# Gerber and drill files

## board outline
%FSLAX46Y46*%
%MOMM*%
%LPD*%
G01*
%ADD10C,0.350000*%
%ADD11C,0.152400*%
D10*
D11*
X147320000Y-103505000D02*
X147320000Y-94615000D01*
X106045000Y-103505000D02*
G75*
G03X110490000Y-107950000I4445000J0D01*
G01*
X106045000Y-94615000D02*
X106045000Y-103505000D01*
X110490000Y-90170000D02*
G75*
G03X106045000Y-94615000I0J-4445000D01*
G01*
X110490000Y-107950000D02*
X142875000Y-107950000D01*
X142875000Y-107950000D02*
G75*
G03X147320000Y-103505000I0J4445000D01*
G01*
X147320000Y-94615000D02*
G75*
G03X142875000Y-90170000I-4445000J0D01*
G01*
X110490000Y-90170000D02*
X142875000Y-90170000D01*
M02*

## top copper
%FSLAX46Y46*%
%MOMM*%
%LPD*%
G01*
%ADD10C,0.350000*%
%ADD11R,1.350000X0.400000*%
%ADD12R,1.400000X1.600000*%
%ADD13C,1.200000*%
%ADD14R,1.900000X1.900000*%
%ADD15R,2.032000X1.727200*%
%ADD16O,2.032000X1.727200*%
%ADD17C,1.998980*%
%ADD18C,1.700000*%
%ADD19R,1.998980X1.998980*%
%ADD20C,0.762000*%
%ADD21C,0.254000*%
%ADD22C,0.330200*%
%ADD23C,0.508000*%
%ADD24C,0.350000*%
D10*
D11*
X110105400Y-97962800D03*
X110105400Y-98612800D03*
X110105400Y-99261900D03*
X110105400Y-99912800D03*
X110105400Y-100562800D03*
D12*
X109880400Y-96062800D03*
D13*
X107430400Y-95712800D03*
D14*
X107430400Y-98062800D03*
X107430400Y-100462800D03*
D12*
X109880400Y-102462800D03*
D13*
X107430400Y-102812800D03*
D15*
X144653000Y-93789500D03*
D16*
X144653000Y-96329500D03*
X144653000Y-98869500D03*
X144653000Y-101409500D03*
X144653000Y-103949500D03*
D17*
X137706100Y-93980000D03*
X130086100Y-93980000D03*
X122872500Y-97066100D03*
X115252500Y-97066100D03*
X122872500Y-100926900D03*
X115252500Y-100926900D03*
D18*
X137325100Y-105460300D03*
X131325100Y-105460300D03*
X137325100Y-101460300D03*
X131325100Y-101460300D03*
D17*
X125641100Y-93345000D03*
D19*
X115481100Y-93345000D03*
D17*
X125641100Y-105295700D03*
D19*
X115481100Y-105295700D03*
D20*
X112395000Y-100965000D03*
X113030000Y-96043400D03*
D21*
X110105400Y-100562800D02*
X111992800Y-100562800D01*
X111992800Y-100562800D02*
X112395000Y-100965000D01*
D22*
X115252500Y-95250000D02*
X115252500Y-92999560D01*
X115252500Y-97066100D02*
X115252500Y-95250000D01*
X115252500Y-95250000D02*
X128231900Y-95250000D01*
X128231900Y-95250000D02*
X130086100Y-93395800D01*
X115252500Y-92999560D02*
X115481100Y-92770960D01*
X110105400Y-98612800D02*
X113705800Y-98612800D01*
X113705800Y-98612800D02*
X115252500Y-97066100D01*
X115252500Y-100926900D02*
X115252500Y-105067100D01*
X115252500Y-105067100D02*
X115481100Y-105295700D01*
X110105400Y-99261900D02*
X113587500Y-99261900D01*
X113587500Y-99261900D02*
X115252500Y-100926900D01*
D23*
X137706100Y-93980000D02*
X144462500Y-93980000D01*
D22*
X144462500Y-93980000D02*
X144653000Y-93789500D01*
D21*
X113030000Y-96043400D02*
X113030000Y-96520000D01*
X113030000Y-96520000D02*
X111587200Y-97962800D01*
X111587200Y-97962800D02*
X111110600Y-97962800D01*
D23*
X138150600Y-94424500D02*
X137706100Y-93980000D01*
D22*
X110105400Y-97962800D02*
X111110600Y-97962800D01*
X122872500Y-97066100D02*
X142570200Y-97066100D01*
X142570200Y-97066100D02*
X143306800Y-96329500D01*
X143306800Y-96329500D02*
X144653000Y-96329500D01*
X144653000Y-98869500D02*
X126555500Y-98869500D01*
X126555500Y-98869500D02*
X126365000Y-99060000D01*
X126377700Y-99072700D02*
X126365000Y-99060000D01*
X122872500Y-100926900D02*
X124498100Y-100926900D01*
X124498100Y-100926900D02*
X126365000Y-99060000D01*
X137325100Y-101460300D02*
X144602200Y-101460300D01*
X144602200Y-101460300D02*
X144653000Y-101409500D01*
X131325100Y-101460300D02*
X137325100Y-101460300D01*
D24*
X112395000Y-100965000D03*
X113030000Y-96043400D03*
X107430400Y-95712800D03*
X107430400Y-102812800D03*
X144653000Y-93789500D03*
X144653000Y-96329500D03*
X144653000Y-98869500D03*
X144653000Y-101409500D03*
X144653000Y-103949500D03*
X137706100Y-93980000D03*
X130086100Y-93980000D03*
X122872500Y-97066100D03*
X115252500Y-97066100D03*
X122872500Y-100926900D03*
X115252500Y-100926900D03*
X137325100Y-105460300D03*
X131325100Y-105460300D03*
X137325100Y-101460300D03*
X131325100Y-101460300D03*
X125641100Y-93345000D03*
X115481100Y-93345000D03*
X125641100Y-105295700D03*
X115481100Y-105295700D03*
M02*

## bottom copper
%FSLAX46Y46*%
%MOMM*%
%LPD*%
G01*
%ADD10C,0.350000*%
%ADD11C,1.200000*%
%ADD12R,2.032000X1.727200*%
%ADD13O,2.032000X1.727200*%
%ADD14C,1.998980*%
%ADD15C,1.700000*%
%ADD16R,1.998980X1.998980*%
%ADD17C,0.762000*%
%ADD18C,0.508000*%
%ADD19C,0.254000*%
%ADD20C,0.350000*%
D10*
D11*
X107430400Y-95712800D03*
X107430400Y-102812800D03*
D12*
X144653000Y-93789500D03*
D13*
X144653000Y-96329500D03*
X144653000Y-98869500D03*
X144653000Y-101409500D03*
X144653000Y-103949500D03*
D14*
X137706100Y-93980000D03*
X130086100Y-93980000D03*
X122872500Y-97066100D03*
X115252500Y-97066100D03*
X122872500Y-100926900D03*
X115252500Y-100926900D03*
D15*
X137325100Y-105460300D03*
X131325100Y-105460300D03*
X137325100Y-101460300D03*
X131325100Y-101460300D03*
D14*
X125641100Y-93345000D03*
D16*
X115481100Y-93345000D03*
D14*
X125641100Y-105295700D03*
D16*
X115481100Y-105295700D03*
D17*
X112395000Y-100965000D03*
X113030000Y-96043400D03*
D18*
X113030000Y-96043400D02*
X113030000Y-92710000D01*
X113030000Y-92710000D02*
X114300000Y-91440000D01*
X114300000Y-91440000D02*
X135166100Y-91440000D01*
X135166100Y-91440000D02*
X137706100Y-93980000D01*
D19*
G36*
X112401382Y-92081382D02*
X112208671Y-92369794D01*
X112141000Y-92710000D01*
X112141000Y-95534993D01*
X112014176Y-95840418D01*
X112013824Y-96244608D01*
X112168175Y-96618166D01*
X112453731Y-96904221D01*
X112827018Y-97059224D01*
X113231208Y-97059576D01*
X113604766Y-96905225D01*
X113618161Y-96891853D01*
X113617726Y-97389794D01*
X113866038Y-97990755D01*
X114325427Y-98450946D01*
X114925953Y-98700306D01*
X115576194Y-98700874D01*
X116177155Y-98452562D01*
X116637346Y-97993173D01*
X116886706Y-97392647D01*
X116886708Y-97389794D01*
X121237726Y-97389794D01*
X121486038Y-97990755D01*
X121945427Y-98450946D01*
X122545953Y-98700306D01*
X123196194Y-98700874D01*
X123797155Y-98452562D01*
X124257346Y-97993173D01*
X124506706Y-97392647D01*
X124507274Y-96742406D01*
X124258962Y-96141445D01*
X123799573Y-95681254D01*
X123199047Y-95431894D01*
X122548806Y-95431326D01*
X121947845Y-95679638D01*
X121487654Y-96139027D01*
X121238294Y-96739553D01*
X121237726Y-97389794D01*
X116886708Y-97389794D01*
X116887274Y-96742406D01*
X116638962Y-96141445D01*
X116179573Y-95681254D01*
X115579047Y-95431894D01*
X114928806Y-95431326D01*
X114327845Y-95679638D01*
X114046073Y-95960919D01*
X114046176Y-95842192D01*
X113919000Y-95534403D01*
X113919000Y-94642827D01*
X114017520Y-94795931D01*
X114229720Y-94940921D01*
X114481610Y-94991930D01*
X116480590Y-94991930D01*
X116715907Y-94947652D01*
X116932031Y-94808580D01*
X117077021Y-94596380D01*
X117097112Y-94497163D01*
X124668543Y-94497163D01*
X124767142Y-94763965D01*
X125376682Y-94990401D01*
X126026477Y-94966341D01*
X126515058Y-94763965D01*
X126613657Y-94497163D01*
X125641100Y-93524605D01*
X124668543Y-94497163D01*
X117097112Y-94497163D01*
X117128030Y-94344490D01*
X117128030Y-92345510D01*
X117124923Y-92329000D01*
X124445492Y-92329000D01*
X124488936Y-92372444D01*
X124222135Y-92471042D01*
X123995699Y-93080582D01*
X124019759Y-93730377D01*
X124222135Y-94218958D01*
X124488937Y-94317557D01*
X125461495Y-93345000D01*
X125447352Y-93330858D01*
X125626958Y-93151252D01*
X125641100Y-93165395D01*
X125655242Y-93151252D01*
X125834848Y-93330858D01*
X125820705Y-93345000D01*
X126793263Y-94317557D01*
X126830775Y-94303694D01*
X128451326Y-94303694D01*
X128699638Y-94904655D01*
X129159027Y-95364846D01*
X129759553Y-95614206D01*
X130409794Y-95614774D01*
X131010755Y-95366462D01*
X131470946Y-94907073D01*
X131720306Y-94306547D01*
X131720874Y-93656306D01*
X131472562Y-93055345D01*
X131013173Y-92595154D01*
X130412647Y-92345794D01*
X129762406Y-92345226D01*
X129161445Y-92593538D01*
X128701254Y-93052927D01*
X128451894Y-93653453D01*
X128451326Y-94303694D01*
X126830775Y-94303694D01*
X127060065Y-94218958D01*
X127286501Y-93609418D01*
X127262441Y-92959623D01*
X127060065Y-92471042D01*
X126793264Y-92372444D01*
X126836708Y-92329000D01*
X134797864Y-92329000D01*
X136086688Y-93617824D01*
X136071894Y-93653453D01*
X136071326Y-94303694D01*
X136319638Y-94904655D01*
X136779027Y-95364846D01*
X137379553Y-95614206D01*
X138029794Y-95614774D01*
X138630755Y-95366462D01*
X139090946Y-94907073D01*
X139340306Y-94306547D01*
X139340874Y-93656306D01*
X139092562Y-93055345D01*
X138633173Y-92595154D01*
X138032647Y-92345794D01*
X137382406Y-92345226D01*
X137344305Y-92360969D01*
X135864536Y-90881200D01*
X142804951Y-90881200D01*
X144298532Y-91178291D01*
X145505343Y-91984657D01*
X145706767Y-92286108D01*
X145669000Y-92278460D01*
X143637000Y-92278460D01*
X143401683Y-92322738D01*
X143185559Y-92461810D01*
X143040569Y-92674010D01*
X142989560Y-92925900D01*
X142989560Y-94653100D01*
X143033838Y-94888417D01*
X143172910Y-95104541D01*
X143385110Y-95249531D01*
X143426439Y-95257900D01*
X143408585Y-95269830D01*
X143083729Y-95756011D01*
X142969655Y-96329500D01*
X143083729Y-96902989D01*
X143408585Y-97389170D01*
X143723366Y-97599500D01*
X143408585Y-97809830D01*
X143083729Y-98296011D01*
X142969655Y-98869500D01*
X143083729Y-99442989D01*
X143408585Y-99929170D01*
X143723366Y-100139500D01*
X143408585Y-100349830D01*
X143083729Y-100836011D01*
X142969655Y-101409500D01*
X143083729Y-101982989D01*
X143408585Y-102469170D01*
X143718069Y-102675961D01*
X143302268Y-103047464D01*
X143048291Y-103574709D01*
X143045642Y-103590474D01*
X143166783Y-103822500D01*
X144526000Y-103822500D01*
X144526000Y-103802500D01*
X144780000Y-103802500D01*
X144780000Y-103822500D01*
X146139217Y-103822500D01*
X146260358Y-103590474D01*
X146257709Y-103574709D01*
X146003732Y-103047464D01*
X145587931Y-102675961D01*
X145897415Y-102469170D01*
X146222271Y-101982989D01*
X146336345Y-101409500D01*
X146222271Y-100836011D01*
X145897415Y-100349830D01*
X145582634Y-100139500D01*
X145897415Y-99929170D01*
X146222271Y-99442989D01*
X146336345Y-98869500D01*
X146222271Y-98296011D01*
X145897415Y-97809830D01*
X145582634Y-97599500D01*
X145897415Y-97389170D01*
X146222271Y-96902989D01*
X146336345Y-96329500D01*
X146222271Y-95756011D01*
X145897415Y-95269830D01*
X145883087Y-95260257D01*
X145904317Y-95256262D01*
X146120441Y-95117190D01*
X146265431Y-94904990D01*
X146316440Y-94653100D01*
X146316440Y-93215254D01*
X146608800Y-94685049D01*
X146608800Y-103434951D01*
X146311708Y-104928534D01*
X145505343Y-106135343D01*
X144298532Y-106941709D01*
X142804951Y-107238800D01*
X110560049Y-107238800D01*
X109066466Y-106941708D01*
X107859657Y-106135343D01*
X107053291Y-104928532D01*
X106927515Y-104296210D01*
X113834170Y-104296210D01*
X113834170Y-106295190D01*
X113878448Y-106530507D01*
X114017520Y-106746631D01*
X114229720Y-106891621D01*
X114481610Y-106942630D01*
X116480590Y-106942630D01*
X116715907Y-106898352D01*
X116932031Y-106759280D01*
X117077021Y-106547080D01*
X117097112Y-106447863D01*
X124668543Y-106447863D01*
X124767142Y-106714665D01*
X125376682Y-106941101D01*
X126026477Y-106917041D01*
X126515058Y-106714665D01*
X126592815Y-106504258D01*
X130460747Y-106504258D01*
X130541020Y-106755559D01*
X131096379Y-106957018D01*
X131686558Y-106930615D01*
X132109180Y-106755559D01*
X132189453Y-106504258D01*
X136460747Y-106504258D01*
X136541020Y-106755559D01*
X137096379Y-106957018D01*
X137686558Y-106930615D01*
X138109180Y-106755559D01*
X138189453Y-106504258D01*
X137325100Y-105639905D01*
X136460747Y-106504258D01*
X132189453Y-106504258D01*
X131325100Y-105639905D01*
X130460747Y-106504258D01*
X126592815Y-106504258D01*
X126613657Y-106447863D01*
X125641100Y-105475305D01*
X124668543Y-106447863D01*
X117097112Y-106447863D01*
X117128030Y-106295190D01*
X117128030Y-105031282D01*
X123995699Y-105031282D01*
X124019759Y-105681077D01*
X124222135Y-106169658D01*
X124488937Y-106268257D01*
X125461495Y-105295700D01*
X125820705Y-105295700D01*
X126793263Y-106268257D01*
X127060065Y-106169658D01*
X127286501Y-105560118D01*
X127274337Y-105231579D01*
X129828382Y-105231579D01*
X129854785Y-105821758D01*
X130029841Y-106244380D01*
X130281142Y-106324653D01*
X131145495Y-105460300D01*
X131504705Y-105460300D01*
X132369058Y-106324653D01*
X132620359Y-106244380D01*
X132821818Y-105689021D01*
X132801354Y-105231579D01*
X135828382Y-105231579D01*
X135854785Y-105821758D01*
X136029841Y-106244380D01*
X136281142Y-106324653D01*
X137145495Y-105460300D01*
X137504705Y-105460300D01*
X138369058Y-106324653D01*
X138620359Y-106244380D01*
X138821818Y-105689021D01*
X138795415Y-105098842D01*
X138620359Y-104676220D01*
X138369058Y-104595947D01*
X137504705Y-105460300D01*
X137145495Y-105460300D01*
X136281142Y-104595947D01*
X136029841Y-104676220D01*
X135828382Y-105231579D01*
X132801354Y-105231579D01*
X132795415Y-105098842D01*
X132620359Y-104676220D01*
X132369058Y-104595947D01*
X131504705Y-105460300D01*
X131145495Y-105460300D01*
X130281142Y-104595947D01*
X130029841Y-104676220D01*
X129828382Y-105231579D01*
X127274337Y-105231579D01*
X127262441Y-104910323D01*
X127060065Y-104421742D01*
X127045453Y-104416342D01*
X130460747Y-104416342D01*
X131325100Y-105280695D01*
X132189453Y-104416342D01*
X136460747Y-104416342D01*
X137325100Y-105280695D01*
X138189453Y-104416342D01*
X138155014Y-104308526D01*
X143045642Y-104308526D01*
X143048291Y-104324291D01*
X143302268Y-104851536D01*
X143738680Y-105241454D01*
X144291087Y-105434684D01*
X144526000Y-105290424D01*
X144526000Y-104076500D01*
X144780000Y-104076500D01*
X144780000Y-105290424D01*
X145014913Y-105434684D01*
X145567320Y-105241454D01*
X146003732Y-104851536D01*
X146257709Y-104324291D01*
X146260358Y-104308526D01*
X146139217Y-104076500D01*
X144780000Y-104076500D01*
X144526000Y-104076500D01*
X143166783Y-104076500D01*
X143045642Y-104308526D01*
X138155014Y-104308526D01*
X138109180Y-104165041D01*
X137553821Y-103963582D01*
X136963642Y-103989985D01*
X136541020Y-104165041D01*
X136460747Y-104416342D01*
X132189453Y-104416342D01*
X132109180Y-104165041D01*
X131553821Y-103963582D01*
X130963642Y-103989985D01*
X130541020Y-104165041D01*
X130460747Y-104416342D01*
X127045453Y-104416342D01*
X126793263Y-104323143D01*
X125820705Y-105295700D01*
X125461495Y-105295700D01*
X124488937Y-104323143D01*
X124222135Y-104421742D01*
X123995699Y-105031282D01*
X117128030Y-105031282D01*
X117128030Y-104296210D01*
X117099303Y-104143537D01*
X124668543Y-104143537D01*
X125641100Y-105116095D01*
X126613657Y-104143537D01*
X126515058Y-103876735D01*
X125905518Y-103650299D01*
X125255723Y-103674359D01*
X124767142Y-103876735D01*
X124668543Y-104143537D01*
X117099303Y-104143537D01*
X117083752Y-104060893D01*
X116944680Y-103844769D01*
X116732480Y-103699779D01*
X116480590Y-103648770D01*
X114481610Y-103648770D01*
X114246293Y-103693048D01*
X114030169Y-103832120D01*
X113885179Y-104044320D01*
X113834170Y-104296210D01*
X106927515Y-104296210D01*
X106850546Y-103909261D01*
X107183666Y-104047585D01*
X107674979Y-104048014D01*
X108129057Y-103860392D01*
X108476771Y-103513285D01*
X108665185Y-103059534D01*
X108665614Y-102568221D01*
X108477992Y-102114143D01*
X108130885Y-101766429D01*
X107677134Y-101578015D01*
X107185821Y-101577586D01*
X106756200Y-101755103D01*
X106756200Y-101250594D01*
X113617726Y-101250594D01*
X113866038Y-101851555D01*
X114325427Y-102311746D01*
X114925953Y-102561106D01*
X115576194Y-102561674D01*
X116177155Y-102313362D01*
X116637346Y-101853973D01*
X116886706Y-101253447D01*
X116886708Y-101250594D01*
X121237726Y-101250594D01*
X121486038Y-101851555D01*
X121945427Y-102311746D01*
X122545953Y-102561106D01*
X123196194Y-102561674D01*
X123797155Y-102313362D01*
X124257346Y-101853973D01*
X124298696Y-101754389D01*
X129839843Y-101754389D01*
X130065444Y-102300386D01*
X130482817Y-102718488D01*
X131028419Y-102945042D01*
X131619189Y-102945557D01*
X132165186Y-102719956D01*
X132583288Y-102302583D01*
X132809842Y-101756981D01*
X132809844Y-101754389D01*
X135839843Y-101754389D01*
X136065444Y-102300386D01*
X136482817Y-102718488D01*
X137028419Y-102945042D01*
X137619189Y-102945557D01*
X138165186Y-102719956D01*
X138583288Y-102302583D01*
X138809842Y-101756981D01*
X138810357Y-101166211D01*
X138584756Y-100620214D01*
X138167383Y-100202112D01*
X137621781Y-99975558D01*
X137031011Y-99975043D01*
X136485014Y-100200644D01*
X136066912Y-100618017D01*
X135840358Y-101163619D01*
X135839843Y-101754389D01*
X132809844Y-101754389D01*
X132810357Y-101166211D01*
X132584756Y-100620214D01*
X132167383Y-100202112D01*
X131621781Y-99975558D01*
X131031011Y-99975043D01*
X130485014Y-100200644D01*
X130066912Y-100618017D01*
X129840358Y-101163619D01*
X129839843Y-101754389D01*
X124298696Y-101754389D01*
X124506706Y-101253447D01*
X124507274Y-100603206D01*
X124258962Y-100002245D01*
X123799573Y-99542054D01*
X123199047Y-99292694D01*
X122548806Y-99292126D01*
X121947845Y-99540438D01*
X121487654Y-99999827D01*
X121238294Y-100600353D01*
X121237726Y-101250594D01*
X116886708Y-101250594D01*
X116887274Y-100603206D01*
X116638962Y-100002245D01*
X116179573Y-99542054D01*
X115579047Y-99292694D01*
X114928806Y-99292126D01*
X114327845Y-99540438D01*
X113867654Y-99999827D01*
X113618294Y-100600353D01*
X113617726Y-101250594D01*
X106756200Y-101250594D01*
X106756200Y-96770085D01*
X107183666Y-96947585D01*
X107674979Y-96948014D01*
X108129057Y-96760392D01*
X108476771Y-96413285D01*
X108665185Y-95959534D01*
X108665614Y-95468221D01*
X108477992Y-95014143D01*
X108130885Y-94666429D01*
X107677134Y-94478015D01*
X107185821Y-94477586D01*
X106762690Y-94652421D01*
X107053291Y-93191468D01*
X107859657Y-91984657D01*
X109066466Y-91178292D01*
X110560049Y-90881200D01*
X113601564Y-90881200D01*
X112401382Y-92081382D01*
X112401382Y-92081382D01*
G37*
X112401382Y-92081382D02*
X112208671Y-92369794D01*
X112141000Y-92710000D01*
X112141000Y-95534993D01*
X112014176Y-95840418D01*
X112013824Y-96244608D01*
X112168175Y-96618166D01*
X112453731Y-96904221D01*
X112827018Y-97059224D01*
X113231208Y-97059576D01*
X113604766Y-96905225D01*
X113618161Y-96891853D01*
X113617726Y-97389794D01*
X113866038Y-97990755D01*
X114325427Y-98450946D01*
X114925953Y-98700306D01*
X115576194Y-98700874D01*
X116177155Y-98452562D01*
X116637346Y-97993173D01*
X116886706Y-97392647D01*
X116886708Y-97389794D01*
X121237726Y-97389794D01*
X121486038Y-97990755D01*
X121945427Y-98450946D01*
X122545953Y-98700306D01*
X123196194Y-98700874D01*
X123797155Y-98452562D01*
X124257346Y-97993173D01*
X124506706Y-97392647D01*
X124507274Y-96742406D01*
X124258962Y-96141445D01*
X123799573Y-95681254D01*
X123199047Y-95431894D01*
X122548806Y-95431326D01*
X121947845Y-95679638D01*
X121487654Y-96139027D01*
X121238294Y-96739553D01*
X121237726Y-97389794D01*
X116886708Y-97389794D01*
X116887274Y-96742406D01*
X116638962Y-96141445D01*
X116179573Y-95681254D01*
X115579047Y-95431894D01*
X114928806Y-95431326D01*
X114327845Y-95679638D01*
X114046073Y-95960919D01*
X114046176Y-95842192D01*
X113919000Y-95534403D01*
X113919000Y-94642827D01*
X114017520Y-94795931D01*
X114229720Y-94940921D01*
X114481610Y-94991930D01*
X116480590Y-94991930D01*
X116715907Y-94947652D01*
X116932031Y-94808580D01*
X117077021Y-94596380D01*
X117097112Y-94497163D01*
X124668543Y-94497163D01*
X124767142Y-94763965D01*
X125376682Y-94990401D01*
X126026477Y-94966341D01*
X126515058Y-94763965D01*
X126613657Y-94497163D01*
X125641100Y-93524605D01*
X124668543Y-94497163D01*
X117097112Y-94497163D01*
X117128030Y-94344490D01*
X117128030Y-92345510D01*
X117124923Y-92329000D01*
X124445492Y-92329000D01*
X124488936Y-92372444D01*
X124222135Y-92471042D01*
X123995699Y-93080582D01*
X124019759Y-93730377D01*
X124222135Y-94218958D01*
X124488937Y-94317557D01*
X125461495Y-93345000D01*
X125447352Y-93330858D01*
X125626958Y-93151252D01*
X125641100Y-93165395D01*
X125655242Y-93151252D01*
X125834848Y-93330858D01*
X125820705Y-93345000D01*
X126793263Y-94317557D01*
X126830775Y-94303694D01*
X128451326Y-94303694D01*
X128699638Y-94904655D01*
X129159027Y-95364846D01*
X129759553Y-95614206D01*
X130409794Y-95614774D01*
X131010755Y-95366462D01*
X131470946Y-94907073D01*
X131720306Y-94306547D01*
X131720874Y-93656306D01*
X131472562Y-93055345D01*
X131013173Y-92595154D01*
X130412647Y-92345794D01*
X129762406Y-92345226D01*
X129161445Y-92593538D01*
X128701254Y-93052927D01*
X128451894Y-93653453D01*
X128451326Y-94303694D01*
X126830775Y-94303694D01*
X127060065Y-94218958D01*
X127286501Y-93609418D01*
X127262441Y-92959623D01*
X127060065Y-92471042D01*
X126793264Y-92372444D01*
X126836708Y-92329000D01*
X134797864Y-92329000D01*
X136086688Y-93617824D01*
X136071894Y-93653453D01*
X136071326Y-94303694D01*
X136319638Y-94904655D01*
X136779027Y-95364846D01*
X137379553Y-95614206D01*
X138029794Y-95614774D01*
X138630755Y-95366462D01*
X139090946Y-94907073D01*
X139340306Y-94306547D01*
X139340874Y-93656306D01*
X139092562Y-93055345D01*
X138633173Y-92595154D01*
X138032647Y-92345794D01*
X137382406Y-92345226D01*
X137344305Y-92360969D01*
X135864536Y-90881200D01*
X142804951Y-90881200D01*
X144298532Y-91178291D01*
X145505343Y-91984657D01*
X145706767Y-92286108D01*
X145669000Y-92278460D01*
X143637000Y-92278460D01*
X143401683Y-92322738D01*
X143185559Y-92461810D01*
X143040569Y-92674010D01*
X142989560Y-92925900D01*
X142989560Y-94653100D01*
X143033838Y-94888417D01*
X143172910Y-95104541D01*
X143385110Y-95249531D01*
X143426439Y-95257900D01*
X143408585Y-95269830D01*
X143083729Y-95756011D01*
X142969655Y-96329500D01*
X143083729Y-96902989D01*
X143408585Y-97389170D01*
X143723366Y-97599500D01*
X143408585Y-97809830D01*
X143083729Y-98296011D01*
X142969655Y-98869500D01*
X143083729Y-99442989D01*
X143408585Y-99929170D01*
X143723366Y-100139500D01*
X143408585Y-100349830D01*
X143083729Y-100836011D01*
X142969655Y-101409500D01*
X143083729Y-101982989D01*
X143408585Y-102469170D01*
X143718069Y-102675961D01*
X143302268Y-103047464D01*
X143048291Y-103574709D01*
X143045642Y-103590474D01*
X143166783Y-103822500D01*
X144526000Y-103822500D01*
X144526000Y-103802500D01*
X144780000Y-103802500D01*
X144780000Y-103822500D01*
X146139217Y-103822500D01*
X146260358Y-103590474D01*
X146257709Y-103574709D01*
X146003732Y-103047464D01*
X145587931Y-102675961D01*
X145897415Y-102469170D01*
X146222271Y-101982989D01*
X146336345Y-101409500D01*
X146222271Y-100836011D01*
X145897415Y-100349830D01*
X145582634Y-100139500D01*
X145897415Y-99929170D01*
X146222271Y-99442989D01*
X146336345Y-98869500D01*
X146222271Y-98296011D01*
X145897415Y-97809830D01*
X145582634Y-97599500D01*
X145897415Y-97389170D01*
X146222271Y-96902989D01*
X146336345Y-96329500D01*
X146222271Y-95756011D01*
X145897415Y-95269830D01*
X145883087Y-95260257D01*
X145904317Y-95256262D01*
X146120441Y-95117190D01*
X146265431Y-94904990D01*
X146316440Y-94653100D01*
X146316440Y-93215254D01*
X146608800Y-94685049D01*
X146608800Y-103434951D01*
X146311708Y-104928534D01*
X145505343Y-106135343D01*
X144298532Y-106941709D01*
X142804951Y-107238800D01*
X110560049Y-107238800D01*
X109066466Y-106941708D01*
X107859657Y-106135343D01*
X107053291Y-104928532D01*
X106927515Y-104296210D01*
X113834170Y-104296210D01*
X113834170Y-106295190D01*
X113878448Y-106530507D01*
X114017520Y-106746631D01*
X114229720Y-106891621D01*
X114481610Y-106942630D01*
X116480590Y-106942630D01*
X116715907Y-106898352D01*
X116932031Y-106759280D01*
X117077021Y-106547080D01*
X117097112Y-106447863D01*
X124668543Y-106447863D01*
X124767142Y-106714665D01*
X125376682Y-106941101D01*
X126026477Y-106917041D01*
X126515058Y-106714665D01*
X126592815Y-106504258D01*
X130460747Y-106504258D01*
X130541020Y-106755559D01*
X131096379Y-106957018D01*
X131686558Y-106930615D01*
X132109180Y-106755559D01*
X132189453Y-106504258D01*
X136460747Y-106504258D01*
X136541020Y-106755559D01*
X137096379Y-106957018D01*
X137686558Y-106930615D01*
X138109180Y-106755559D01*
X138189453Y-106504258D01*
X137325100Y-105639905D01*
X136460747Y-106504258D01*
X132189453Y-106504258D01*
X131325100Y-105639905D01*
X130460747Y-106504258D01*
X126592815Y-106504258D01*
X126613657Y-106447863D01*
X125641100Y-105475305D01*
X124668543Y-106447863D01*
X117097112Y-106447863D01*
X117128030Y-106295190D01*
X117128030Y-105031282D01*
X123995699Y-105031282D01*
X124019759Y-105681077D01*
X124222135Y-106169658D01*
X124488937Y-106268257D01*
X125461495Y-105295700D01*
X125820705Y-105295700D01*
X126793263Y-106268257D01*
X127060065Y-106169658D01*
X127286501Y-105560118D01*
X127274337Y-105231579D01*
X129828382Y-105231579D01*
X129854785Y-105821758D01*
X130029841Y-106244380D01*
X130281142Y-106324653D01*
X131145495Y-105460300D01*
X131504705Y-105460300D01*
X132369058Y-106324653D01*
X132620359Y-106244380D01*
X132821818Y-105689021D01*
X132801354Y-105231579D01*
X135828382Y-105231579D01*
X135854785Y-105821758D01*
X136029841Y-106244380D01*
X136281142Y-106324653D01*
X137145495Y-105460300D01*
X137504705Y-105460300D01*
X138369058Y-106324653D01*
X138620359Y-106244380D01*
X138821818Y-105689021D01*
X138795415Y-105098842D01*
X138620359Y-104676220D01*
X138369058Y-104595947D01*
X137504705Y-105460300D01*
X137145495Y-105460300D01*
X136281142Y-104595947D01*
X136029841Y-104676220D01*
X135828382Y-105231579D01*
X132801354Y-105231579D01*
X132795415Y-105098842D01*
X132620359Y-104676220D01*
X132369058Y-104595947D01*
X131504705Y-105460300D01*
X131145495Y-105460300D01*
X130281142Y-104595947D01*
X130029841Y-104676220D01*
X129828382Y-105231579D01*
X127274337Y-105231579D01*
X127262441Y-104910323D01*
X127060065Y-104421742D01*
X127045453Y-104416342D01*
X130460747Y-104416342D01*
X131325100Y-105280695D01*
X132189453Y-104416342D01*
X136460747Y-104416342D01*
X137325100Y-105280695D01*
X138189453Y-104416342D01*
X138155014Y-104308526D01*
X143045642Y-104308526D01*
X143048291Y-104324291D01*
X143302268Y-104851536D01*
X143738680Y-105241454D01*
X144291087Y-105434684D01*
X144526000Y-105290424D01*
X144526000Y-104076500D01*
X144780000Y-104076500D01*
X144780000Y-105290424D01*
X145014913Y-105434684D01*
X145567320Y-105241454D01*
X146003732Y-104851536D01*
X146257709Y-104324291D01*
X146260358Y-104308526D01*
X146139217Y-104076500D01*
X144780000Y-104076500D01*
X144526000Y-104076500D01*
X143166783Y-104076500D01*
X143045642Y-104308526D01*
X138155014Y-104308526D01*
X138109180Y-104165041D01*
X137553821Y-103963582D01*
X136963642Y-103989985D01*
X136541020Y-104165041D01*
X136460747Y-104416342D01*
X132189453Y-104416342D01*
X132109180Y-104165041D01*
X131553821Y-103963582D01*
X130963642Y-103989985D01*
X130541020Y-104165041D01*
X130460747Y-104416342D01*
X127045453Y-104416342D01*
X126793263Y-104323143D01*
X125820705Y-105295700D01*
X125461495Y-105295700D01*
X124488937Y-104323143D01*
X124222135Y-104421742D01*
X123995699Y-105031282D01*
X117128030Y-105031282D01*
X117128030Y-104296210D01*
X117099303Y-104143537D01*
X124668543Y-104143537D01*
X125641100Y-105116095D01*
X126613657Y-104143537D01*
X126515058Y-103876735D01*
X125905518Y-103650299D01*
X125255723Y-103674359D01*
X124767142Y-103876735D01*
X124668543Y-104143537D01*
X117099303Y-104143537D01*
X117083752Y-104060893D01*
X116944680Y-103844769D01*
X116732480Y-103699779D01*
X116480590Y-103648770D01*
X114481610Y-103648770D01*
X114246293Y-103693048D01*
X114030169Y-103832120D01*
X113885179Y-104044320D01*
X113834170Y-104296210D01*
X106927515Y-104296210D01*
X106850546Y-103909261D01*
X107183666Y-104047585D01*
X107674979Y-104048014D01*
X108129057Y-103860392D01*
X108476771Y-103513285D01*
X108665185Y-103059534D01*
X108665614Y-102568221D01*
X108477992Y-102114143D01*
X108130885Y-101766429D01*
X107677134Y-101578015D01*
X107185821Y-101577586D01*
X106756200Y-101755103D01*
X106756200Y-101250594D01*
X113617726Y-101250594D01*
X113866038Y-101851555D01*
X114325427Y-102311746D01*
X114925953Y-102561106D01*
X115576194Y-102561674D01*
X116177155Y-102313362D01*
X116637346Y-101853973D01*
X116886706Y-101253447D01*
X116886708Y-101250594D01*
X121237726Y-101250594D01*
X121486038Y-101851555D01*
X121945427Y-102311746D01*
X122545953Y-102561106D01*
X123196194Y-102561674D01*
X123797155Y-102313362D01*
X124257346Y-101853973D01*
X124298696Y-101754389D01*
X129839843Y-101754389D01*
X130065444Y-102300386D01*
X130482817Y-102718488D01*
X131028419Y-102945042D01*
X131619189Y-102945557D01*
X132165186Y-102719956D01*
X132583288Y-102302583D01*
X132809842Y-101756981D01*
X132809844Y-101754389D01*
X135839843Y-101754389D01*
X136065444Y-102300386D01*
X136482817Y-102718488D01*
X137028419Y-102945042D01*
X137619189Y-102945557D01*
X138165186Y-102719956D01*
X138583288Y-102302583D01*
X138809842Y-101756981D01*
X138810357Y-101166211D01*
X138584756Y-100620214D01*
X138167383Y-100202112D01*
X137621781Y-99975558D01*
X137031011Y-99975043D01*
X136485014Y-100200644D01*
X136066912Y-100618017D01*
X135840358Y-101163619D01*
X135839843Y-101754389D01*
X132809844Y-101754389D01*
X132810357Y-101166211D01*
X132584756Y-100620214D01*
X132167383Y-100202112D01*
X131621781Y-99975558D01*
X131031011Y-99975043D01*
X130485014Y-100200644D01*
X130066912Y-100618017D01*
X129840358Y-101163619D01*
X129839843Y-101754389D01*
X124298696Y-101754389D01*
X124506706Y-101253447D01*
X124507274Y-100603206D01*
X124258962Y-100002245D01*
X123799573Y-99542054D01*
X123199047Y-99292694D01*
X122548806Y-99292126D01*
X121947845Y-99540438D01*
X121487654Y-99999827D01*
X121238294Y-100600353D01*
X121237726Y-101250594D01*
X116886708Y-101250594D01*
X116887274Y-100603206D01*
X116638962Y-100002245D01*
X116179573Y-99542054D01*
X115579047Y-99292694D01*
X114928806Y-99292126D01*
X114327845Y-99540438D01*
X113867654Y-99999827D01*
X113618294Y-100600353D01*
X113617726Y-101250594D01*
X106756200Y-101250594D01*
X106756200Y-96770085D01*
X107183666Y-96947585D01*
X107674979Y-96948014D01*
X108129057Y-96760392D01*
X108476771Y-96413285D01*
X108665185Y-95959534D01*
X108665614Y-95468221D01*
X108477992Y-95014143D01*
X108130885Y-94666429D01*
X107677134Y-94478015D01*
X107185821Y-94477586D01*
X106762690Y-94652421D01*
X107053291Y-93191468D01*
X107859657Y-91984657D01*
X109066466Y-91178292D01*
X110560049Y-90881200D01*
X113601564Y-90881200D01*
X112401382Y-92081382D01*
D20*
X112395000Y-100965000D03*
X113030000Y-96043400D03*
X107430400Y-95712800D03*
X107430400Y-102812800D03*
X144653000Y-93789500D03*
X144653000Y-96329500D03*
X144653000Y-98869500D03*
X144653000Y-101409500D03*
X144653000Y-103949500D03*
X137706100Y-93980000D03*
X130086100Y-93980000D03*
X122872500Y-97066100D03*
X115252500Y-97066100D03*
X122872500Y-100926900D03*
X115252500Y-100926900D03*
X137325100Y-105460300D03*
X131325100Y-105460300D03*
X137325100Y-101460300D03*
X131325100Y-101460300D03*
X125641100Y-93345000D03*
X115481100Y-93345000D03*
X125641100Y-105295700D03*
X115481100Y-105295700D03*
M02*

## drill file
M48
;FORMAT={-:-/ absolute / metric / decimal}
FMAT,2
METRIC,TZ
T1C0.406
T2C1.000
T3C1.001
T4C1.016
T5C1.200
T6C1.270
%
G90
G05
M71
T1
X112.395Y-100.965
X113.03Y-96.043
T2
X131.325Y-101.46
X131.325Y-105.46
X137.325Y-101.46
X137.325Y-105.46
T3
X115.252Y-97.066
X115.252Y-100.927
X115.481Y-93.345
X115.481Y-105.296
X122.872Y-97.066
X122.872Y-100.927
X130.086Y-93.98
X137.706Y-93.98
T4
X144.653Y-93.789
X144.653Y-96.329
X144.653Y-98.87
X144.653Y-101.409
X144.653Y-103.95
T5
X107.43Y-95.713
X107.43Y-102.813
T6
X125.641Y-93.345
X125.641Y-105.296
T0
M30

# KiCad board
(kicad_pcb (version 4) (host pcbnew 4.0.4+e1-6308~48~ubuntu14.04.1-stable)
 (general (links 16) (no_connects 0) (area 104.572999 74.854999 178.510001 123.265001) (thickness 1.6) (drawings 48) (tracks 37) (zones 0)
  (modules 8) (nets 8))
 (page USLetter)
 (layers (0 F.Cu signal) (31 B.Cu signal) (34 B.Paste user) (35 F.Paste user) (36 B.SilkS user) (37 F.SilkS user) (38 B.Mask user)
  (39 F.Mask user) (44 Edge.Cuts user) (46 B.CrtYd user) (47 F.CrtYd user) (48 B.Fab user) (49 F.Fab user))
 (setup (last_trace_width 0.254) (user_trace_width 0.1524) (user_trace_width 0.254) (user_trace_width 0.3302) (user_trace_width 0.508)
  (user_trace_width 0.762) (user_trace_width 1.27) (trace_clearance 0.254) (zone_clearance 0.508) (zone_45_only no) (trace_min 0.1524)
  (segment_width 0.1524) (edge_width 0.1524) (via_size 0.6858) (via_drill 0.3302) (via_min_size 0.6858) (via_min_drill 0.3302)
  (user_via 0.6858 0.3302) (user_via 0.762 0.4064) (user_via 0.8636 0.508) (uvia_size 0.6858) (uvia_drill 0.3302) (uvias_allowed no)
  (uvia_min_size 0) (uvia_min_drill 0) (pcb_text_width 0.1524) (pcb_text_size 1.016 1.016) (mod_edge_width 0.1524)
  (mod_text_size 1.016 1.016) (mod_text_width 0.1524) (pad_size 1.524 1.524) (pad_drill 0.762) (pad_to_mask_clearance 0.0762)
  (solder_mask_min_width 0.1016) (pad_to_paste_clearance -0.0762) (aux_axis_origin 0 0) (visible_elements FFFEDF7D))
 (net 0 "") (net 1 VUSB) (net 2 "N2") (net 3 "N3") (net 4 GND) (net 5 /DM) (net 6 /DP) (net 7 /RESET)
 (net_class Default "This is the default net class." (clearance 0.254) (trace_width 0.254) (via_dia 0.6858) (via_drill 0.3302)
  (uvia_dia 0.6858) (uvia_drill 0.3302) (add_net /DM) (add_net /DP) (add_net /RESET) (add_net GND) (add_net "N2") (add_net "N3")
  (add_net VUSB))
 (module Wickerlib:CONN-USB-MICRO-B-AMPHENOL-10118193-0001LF (layer F.Cu) (at 107.4304 99.2628 270)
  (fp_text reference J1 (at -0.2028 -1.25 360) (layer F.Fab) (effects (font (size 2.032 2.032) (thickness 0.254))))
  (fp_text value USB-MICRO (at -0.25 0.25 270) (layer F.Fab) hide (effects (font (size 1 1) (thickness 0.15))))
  (pad 1 smd rect (at -1.3 -2.675) (size 1.35 0.4) (layers F.Cu F.Paste F.Mask) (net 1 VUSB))
  (pad 2 smd rect (at -0.65 -2.675) (size 1.35 0.4) (layers F.Cu F.Paste F.Mask) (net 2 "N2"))
  (pad 3 smd rect (at -0.0009 -2.675) (size 1.35 0.4) (layers F.Cu F.Paste F.Mask) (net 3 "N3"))
  (pad 4 smd rect (at 0.65 -2.675) (size 1.35 0.4) (layers F.Cu F.Paste F.Mask))
  (pad 5 smd rect (at 1.3 -2.675) (size 1.35 0.4) (layers F.Cu F.Paste F.Mask) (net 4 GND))
  (pad 6 smd rect (at -3.2 -2.45) (size 1.4 1.6) (layers F.Cu F.Paste F.Mask))
  (pad 6 thru_hole circle (at -3.55 0) (size 1.2 1.2) (drill 1.2) (layers *.Cu *.Mask F.SilkS))
  (pad 6 smd rect (at -1.2 0) (size 1.9 1.9) (layers F.Cu F.Paste F.Mask))
  (pad 6 smd rect (at 1.2 0) (size 1.9 1.9) (layers F.Cu F.Paste F.Mask))
  (pad 6 smd rect (at 3.2 -2.45) (size 1.4 1.6) (layers F.Cu F.Paste F.Mask))
  (pad 6 thru_hole circle (at 3.55 0) (size 1.2 1.2) (drill 1.2) (layers *.Cu *.Mask F.SilkS)))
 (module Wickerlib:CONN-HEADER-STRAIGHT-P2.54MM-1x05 (layer F.Cu) (at 144.653 93.7895)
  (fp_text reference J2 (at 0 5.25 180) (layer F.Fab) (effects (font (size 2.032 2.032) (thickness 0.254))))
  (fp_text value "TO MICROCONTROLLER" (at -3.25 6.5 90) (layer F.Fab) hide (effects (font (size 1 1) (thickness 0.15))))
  (pad 1 thru_hole rect (at 0 0) (size 2.032 1.7272) (drill 1.016) (layers *.Cu *.Mask F.SilkS) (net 1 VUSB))
  (pad 2 thru_hole oval (at 0 2.54) (size 2.032 1.7272) (drill 1.016) (layers *.Cu *.Mask F.SilkS) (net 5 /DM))
  (pad 3 thru_hole oval (at 0 5.08) (size 2.032 1.7272) (drill 1.016) (layers *.Cu *.Mask F.SilkS) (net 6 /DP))
  (pad 4 thru_hole oval (at 0 7.62) (size 2.032 1.7272) (drill 1.016) (layers *.Cu *.Mask F.SilkS) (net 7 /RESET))
  (pad 5 thru_hole oval (at 0 10.16) (size 2.032 1.7272) (drill 1.016) (layers *.Cu *.Mask F.SilkS) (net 4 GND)))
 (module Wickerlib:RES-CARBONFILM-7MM (layer F.Cu) (at 137.7061 93.98 180)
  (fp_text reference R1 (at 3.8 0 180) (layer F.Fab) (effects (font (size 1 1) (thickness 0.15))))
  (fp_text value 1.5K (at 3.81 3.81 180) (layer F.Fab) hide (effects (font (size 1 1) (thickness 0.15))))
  (pad 1 thru_hole circle (at 0 0 180) (size 1.99898 1.99898) (drill 1.00076) (layers *.Cu *.SilkS *.Mask) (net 1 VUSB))
  (pad 2 thru_hole circle (at 7.62 0 180) (size 1.99898 1.99898) (drill 1.00076) (layers *.Cu *.SilkS *.Mask) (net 2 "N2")))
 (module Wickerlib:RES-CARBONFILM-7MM (layer F.Cu) (at 122.8725 97.0661 180)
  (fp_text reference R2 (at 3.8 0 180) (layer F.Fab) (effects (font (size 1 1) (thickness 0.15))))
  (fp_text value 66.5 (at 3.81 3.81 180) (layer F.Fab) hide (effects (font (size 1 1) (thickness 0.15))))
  (pad 1 thru_hole circle (at 0 0 180) (size 1.99898 1.99898) (drill 1.00076) (layers *.Cu *.SilkS *.Mask) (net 5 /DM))
  (pad 2 thru_hole circle (at 7.62 0 180) (size 1.99898 1.99898) (drill 1.00076) (layers *.Cu *.SilkS *.Mask) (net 2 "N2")))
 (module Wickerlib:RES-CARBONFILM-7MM (layer F.Cu) (at 122.8725 100.9269 180)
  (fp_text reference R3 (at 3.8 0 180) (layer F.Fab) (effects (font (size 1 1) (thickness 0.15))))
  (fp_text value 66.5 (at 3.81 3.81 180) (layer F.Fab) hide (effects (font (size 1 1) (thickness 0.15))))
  (pad 1 thru_hole circle (at 0 0 180) (size 1.99898 1.99898) (drill 1.00076) (layers *.Cu *.SilkS *.Mask) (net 6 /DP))
  (pad 2 thru_hole circle (at 7.62 0 180) (size 1.99898 1.99898) (drill 1.00076) (layers *.Cu *.SilkS *.Mask) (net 3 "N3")))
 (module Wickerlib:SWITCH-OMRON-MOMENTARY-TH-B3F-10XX (layer F.Cu) (at 131.3251 101.4603)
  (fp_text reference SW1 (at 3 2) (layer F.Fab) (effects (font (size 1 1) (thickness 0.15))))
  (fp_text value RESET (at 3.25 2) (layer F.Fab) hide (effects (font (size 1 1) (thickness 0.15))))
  (pad 4 thru_hole circle (at 6 4) (size 1.7 1.7) (drill 1) (layers *.Cu *.Mask) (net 4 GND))
  (pad 3 thru_hole circle (at 0 4) (size 1.7 1.7) (drill 1) (layers *.Cu *.Mask) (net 4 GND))
  (pad 2 thru_hole circle (at 6 0) (size 1.7 1.7) (drill 1) (layers *.Cu *.Mask) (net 7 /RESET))
  (pad 1 thru_hole circle (at 0 0) (size 1.7 1.7) (drill 1) (layers *.Cu *.Mask) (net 7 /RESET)))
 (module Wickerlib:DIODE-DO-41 (layer F.Cu) (at 115.4811 93.34754)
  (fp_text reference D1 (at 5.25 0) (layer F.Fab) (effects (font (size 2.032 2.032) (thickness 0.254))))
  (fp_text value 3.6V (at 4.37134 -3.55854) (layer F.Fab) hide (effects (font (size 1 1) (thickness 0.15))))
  (pad 2 thru_hole circle (at 10.16 -0.00254 180) (size 1.99898 1.99898) (drill 1.27) (layers *.Cu *.Mask F.SilkS) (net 4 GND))
  (pad 1 thru_hole rect (at 0 -0.00254 180) (size 1.99898 1.99898) (drill 1.00076) (layers *.Cu *.Mask F.SilkS) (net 2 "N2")))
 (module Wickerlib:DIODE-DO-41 (layer F.Cu) (at 115.4811 105.29824)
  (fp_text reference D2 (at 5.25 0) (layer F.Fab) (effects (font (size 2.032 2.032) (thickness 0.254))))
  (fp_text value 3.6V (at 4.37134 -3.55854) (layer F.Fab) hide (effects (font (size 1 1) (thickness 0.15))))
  (pad 2 thru_hole circle (at 10.16 -0.00254 180) (size 1.99898 1.99898) (drill 1.27) (layers *.Cu *.Mask F.SilkS) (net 4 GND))
  (pad 1 thru_hole rect (at 0 -0.00254 180) (size 1.99898 1.99898) (drill 1.00076) (layers *.Cu *.Mask F.SilkS) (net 3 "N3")))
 (gr_line (start 147.32 103.505) (end 147.32 94.615) (layer Edge.Cuts) (width 0.1524))
 (gr_arc (start 110.49 103.505) (end 110.49 107.95) (angle 90) (layer Edge.Cuts) (width 0.1524))
 (gr_line (start 106.045 94.615) (end 106.045 103.505) (layer Edge.Cuts) (width 0.1524))
 (gr_arc (start 110.49 94.615) (end 106.045 94.615) (angle 90) (layer Edge.Cuts) (width 0.1524))
 (gr_line (start 110.49 107.95) (end 142.875 107.95) (layer Edge.Cuts) (width 0.1524))
 (gr_arc (start 142.875 103.505) (end 147.32 103.505) (angle 90) (layer Edge.Cuts) (width 0.1524))
 (gr_arc (start 142.875 94.615) (end 142.875 90.17) (angle 90) (layer Edge.Cuts) (width 0.1524))
 (gr_line (start 110.49 90.17) (end 142.875 90.17) (layer Edge.Cuts) (width 0.1524))
 (segment (start 110.1054 100.5628) (end 111.9928 100.5628) (width 0.254) (layer F.Cu) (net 4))
 (segment (start 111.9928 100.5628) (end 112.395 100.965) (width 0.254) (layer F.Cu) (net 4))
 (via (at 112.395 100.965) (size 0.762) (drill 0.4064) (layers F.Cu B.Cu) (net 4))
 (segment (start 115.2525 95.25) (end 115.2525 92.99956) (width 0.3302) (layer F.Cu) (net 2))
 (segment (start 115.2525 97.0661) (end 115.2525 95.25) (width 0.3302) (layer F.Cu) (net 2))
 (segment (start 115.2525 95.25) (end 128.2319 95.25) (width 0.3302) (layer F.Cu) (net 2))
 (segment (start 128.2319 95.25) (end 130.0861 93.3958) (width 0.3302) (layer F.Cu) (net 2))
 (segment (start 115.2525 92.99956) (end 115.4811 92.77096) (width 0.3302) (layer F.Cu) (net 2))
 (segment (start 110.1054 98.6128) (end 113.7058 98.6128) (width 0.3302) (layer F.Cu) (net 2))
 (segment (start 113.7058 98.6128) (end 115.2525 97.0661) (width 0.3302) (layer F.Cu) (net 2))
 (segment (start 115.2525 100.9269) (end 115.2525 105.0671) (width 0.3302) (layer F.Cu) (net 3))
 (segment (start 115.2525 105.0671) (end 115.4811 105.2957) (width 0.3302) (layer F.Cu) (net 3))
 (segment (start 110.1054 99.2619) (end 113.5875 99.2619) (width 0.3302) (layer F.Cu) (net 3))
 (segment (start 113.5875 99.2619) (end 115.2525 100.9269) (width 0.3302) (layer F.Cu) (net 3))
 (segment (start 137.7061 93.98) (end 144.4625 93.98) (width 0.508) (layer F.Cu) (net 1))
 (segment (start 144.4625 93.98) (end 144.653 93.7895) (width 0.3302) (layer F.Cu) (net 1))
 (segment (start 113.03 96.0434) (end 113.03 96.52) (width 0.254) (layer F.Cu) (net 1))
 (segment (start 113.03 96.52) (end 111.5872 97.9628) (width 0.254) (layer F.Cu) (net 1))
 (segment (start 111.5872 97.9628) (end 111.1106 97.9628) (width 0.254) (layer F.Cu) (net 1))
 (segment (start 138.1506 94.4245) (end 137.7061 93.98) (width 0.508) (layer F.Cu) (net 1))
 (segment (start 113.03 96.0434) (end 113.03 92.71) (width 0.508) (layer B.Cu) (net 1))
 (segment (start 113.03 92.71) (end 114.3 91.44) (width 0.508) (layer B.Cu) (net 1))
 (segment (start 114.3 91.44) (end 135.1661 91.44) (width 0.508) (layer B.Cu) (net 1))
 (segment (start 135.1661 91.44) (end 137.7061 93.98) (width 0.508) (layer B.Cu) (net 1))
 (via (at 113.03 96.0434) (size 0.762) (drill 0.4064) (layers F.Cu B.Cu) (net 1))
 (segment (start 110.1054 97.9628) (end 111.1106 97.9628) (width 0.3302) (layer F.Cu) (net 1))
 (segment (start 122.8725 97.0661) (end 142.5702 97.0661) (width 0.3302) (layer F.Cu) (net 5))
 (segment (start 142.5702 97.0661) (end 143.3068 96.3295) (width 0.3302) (layer F.Cu) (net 5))
 (segment (start 143.3068 96.3295) (end 144.653 96.3295) (width 0.3302) (layer F.Cu) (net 5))
 (segment (start 144.653 98.8695) (end 126.5555 98.8695) (width 0.3302) (layer F.Cu) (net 6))
 (segment (start 126.5555 98.8695) (end 126.365 99.06) (width 0.3302) (layer F.Cu) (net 6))
 (segment (start 126.3777 99.0727) (end 126.365 99.06) (width 0.3302) (layer F.Cu) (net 6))
 (segment (start 122.8725 100.9269) (end 124.4981 100.9269) (width 0.3302) (layer F.Cu) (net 6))
 (segment (start 124.4981 100.9269) (end 126.365 99.06) (width 0.3302) (layer F.Cu) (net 6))
 (segment (start 137.3251 101.4603) (end 144.6022 101.4603) (width 0.3302) (layer F.Cu) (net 7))
 (segment (start 144.6022 101.4603) (end 144.653 101.4095) (width 0.3302) (layer F.Cu) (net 7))
 (segment (start 131.3251 101.4603) (end 137.3251 101.4603) (width 0.3302) (layer F.Cu) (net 7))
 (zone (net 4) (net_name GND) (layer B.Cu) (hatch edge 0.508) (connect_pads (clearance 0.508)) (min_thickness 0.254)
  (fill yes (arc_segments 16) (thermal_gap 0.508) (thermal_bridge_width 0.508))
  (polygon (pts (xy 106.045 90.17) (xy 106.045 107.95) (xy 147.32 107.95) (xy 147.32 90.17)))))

